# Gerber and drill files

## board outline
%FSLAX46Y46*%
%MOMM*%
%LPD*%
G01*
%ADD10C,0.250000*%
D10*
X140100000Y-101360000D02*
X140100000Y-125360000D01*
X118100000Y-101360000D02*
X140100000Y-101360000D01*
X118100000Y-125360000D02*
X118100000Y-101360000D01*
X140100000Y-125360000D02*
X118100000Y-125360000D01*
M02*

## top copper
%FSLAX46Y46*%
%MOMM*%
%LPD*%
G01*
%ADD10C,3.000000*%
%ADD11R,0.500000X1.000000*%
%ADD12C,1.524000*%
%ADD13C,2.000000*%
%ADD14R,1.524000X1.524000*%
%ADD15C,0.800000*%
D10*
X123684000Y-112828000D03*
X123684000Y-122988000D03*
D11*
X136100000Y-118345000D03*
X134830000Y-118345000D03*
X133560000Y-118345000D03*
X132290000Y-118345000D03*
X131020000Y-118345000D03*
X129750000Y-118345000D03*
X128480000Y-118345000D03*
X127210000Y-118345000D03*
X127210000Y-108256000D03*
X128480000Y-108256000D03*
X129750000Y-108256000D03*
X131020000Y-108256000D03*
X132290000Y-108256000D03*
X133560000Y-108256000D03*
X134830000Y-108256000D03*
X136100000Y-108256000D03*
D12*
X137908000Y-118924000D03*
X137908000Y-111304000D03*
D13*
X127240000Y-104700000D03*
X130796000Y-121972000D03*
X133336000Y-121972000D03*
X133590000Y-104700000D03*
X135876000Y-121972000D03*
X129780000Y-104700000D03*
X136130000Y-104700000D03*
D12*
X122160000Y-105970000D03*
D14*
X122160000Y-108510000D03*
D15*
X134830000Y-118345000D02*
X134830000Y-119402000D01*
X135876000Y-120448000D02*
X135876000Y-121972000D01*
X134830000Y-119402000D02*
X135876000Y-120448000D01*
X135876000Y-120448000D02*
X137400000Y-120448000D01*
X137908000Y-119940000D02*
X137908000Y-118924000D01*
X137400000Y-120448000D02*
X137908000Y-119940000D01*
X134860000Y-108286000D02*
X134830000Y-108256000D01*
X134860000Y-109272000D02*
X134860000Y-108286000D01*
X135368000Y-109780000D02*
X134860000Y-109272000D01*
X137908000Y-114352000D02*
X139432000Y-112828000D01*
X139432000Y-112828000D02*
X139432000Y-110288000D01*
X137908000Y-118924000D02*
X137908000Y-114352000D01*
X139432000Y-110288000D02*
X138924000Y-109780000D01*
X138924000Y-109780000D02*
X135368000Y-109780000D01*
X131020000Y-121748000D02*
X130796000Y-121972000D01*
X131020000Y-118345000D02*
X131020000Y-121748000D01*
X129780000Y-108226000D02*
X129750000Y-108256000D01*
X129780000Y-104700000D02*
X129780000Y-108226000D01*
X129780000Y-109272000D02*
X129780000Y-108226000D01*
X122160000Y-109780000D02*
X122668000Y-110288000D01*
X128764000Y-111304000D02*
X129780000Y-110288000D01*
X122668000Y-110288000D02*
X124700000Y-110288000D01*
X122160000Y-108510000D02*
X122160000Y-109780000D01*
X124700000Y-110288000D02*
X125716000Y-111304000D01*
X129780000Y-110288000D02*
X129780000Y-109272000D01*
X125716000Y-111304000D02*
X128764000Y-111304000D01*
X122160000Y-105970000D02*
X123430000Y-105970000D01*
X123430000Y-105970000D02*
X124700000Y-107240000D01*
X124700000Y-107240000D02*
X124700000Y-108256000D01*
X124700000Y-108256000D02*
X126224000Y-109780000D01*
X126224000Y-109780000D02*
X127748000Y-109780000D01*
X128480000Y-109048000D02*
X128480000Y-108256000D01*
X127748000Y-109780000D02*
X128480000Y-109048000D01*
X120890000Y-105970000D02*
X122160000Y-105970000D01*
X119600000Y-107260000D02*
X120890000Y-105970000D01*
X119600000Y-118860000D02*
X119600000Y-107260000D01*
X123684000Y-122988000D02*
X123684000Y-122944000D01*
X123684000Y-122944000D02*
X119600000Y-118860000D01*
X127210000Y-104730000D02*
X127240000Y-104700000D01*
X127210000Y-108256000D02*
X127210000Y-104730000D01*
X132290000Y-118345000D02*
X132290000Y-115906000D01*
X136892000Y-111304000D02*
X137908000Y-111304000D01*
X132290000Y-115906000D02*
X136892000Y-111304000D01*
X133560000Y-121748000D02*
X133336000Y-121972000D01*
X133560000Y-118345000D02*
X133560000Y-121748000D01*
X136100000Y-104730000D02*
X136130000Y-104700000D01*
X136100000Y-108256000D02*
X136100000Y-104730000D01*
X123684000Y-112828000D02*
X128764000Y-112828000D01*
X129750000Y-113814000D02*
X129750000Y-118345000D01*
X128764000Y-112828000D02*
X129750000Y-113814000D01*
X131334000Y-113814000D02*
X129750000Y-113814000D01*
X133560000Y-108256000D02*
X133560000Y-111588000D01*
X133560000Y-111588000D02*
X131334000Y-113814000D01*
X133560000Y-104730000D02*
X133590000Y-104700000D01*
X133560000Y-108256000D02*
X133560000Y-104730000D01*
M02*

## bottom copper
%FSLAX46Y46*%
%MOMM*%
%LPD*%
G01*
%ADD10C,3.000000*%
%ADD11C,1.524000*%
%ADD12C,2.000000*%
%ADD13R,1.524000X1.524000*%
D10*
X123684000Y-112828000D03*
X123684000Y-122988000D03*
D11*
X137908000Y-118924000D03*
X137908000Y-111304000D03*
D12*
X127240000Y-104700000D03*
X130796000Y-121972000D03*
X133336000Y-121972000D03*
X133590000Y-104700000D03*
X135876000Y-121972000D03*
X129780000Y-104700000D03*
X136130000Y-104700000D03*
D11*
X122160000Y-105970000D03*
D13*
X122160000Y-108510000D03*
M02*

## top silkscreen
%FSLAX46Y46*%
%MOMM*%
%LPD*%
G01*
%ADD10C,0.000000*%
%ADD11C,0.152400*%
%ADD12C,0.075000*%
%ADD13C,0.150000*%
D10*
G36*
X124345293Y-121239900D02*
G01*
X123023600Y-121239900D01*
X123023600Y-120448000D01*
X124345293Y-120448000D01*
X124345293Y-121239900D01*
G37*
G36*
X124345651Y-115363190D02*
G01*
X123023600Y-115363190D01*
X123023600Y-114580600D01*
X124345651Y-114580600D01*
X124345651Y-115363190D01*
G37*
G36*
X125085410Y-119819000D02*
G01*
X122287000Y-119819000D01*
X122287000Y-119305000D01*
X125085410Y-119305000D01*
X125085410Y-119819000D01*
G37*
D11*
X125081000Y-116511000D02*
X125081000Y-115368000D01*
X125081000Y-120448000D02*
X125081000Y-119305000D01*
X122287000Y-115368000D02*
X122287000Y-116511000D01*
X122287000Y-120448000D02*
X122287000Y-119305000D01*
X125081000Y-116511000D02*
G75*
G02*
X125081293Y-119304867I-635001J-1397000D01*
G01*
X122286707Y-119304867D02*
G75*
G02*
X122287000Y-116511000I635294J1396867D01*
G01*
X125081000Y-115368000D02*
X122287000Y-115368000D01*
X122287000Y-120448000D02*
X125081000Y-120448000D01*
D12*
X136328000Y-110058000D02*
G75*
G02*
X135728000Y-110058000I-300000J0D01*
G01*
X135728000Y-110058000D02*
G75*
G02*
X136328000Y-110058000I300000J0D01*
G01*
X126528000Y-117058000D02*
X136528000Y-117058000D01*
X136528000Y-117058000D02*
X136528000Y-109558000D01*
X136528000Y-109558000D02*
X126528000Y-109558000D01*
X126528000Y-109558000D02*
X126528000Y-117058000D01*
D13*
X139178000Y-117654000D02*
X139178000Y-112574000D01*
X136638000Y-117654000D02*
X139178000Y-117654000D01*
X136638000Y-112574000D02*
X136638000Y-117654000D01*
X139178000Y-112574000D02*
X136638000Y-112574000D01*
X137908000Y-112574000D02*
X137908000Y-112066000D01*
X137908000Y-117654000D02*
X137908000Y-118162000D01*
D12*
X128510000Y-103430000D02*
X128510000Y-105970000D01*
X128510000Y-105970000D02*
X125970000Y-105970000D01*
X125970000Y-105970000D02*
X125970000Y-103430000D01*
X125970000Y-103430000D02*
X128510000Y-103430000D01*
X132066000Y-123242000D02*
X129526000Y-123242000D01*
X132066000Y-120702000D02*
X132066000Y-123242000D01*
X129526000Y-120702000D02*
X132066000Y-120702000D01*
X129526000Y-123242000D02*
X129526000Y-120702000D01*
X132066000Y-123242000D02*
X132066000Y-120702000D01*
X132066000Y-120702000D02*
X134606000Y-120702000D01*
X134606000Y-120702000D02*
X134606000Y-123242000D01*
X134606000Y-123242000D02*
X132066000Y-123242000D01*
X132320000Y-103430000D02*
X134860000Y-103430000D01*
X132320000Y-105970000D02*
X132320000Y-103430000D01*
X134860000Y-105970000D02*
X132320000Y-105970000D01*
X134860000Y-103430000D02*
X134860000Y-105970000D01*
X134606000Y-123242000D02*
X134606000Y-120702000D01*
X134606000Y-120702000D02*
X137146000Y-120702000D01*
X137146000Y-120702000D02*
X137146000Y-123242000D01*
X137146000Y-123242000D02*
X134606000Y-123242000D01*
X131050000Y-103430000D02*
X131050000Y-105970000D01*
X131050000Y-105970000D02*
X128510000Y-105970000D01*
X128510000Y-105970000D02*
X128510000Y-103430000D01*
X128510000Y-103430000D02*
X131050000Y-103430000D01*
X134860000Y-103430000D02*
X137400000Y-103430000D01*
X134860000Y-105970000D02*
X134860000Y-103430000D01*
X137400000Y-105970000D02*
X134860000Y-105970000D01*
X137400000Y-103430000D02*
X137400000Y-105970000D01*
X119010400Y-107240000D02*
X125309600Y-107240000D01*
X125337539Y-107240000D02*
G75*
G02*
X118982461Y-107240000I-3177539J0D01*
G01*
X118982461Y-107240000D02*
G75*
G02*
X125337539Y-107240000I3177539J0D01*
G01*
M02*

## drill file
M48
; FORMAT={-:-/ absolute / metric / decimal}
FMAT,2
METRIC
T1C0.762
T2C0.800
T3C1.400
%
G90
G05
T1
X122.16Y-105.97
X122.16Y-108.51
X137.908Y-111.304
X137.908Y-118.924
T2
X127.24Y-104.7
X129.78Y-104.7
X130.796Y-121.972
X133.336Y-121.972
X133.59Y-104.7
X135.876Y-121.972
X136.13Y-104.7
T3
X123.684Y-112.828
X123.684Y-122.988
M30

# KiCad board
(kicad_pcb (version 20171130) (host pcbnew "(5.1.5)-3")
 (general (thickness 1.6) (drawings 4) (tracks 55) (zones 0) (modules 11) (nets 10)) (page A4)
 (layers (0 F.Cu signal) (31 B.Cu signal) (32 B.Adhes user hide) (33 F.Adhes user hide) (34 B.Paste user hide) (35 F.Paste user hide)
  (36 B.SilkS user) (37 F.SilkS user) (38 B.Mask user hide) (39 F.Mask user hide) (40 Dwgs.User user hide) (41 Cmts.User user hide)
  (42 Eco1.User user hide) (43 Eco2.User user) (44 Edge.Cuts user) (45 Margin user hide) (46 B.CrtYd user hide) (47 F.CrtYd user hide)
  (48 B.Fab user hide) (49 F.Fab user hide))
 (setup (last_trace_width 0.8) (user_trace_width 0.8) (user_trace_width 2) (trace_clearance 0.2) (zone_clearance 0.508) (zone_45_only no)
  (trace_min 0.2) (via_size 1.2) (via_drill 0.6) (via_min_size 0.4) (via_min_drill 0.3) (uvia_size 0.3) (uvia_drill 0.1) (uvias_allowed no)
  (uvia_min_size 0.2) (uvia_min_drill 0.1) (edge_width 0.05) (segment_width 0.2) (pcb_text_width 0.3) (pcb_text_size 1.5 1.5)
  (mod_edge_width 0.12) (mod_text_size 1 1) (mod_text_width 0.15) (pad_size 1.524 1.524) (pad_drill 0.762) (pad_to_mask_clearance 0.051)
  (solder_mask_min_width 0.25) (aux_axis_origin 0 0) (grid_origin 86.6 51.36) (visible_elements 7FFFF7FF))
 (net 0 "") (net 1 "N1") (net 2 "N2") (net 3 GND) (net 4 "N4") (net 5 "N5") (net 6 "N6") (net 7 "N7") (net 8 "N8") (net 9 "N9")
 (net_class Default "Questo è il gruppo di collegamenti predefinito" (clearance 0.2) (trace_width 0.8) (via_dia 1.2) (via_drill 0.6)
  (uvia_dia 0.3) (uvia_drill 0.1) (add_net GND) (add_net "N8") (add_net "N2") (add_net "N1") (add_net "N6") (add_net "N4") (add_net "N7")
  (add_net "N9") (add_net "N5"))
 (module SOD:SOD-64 (layer F.Cu) (at 123.684 117.908 90)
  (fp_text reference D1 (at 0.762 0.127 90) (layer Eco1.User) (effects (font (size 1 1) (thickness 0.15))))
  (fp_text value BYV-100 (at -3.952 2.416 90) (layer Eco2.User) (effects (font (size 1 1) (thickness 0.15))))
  (fp_poly (pts (xy -3.3319 -0.6604) (xy -2.54 -0.6604) (xy -2.54 0.661293) (xy -3.3319 0.661293)) (layer F.SilkS) (width 0))
  (fp_poly (pts (xy 2.54481 -0.6604) (xy 3.3274 -0.6604) (xy 3.3274 0.661651) (xy 2.54481 0.661651)) (layer F.SilkS) (width 0))
  (fp_poly (pts (xy -1.911 -1.397) (xy -1.397 -1.397) (xy -1.397 1.40141) (xy -1.911 1.40141)) (layer F.SilkS) (width 0))
  (fp_line (start 1.397 1.397) (end 2.54 1.397) (layer F.SilkS) (width 0.1524))
  (fp_line (start -2.54 1.397) (end -1.397 1.397) (layer F.SilkS) (width 0.1524))
  (fp_line (start 2.54 -1.397) (end 1.397 -1.397) (layer F.SilkS) (width 0.1524))
  (fp_line (start -2.54 -1.397) (end -1.397 -1.397) (layer F.SilkS) (width 0.1524))
  (fp_arc (start 0 0.761999) (end 1.397 1.397) (angle 131.1) (layer F.SilkS) (width 0.1524))
  (fp_arc (start 0 -0.761999) (end 1.397 -1.397) (angle -131.1) (layer F.SilkS) (width 0.1524))
  (fp_line (start 2.54 1.397) (end 2.54 -1.397) (layer F.SilkS) (width 0.1524))
  (fp_line (start -2.54 -1.397) (end -2.54 1.397) (layer F.SilkS) (width 0.1524))
  (pad 2 thru_hole circle (at 5.08 0 90) (size 3 3) (drill 1.4) (layers *.Cu *.Mask) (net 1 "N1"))
  (pad 1 thru_hole circle (at -5.08 0 90) (size 3 3) (drill 1.4) (layers *.Cu *.Mask) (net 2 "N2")))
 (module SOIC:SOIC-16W (layer F.Cu) (at 136.1 108.256 180)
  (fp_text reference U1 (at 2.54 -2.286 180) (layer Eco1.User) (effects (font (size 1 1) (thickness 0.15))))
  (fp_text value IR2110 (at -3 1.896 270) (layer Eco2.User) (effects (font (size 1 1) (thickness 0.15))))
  (fp_circle (center 0.072 -1.802) (end 0.372 -1.802) (layer F.SilkS) (width 0.075))
  (fp_line (start 9.572 -8.802) (end -0.428 -8.802) (layer F.SilkS) (width 0.075))
  (fp_line (start -0.428 -8.802) (end -0.428 -1.302) (layer F.SilkS) (width 0.075))
  (fp_line (start -0.428 -1.302) (end 9.572 -1.302) (layer F.SilkS) (width 0.075))
  (fp_line (start 9.572 -1.302) (end 9.572 -8.802) (layer F.SilkS) (width 0.075))
  (pad 16 smd rect (at 0 -10.089 180) (size 0.5 1) (layers F.Cu F.Paste F.Mask))
  (pad 15 smd rect (at 1.27 -10.089 180) (size 0.5 1) (layers F.Cu F.Paste F.Mask) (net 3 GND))
  (pad 14 smd rect (at 2.54 -10.089 180) (size 0.5 1) (layers F.Cu F.Paste F.Mask) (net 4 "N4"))
  (pad 13 smd rect (at 3.81 -10.089 180) (size 0.5 1) (layers F.Cu F.Paste F.Mask) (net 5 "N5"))
  (pad 12 smd rect (at 5.08 -10.089 180) (size 0.5 1) (layers F.Cu F.Paste F.Mask) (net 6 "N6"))
  (pad 11 smd rect (at 6.35 -10.089 180) (size 0.5 1) (layers F.Cu F.Paste F.Mask) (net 1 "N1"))
  (pad 10 smd rect (at 7.62 -10.089 180) (size 0.5 1) (layers F.Cu F.Paste F.Mask))
  (pad 9 smd rect (at 8.89 -10.089 180) (size 0.5 1) (layers F.Cu F.Paste F.Mask))
  (pad 8 smd rect (at 8.89 0 180) (size 0.5 1) (layers F.Cu F.Paste F.Mask) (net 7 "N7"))
  (pad 7 smd rect (at 7.62 0 180) (size 0.5 1) (layers F.Cu F.Paste F.Mask) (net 2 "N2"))
  (pad 6 smd rect (at 6.35 0 180) (size 0.5 1) (layers F.Cu F.Paste F.Mask) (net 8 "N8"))
  (pad 5 smd rect (at 5.08 0 180) (size 0.5 1) (layers F.Cu F.Paste F.Mask))
  (pad 4 smd rect (at 3.81 0 180) (size 0.5 1) (layers F.Cu F.Paste F.Mask))
  (pad 3 smd rect (at 2.54 0 180) (size 0.5 1) (layers F.Cu F.Paste F.Mask) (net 1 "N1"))
  (pad 2 smd rect (at 1.27 0 180) (size 0.5 1) (layers F.Cu F.Paste F.Mask) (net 3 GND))
  (pad 1 smd rect (at 0 0 180) (size 0.5 1) (layers F.Cu F.Paste F.Mask) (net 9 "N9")))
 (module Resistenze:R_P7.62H (layer F.Cu) (at 137.908 115.114 270)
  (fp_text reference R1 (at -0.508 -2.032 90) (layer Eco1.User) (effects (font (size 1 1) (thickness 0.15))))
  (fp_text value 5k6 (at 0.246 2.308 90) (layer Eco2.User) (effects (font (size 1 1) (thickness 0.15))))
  (fp_line (start 2.54 -1.27) (end -2.54 -1.27) (layer F.SilkS) (width 0.15))
  (fp_line (start 2.54 1.27) (end 2.54 -1.27) (layer F.SilkS) (width 0.15))
  (fp_line (start -2.54 1.27) (end 2.54 1.27) (layer F.SilkS) (width 0.15))
  (fp_line (start -2.54 -1.27) (end -2.54 1.27) (layer F.SilkS) (width 0.15))
  (fp_line (start -2.54 0) (end -3.048 0) (layer F.SilkS) (width 0.15))
  (fp_line (start 2.54 0) (end 3.048 0) (layer F.SilkS) (width 0.15))
  (pad 2 thru_hole circle (at 3.81 0 270) (size 1.524 1.524) (drill 0.762) (layers *.Cu *.Mask) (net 3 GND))
  (pad 1 thru_hole circle (at -3.81 0 270) (size 1.524 1.524) (drill 0.762) (layers *.Cu *.Mask) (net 5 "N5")))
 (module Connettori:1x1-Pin (layer F.Cu) (at 127.24 104.7 270)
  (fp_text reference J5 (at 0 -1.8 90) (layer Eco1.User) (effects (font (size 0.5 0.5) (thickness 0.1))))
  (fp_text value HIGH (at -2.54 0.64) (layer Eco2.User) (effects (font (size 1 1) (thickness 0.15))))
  (fp_line (start -1.27 -1.27) (end 1.27 -1.27) (layer F.SilkS) (width 0.075))
  (fp_line (start 1.27 -1.27) (end 1.27 1.27) (layer F.SilkS) (width 0.075))
  (fp_line (start 1.27 1.27) (end -1.27 1.27) (layer F.SilkS) (width 0.075))
  (fp_line (start -1.27 1.27) (end -1.27 -1.27) (layer F.SilkS) (width 0.075))
  (pad 1 thru_hole circle (at 0 0 270) (size 2 2) (drill 0.8) (layers *.Cu *.Mask) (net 7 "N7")))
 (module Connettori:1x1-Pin (layer F.Cu) (at 130.796 121.972 90)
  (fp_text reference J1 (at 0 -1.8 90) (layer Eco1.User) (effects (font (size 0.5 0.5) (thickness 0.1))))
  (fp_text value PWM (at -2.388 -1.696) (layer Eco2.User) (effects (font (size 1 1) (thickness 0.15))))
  (fp_line (start -1.27 1.27) (end -1.27 -1.27) (layer F.SilkS) (width 0.075))
  (fp_line (start 1.27 1.27) (end -1.27 1.27) (layer F.SilkS) (width 0.075))
  (fp_line (start 1.27 -1.27) (end 1.27 1.27) (layer F.SilkS) (width 0.075))
  (fp_line (start -1.27 -1.27) (end 1.27 -1.27) (layer F.SilkS) (width 0.075))
  (pad 1 thru_hole circle (at 0 0 90) (size 2 2) (drill 0.8) (layers *.Cu *.Mask) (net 6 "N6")))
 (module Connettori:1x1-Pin (layer F.Cu) (at 133.336 121.972 90)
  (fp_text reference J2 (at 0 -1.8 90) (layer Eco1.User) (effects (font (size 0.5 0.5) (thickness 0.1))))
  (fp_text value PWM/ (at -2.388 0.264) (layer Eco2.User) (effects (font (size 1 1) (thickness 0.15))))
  (fp_line (start -1.27 -1.27) (end 1.27 -1.27) (layer F.SilkS) (width 0.075))
  (fp_line (start 1.27 -1.27) (end 1.27 1.27) (layer F.SilkS) (width 0.075))
  (fp_line (start 1.27 1.27) (end -1.27 1.27) (layer F.SilkS) (width 0.075))
  (fp_line (start -1.27 1.27) (end -1.27 -1.27) (layer F.SilkS) (width 0.075))
  (pad 1 thru_hole circle (at 0 0 90) (size 2 2) (drill 0.8) (layers *.Cu *.Mask) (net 4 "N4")))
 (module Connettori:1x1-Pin (layer F.Cu) (at 133.59 104.7 270)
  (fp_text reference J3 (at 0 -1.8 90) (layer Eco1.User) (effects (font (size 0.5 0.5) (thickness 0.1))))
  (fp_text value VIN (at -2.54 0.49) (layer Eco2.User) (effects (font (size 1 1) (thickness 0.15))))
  (fp_line (start -1.27 1.27) (end -1.27 -1.27) (layer F.SilkS) (width 0.075))
  (fp_line (start 1.27 1.27) (end -1.27 1.27) (layer F.SilkS) (width 0.075))
  (fp_line (start 1.27 -1.27) (end 1.27 1.27) (layer F.SilkS) (width 0.075))
  (fp_line (start -1.27 -1.27) (end 1.27 -1.27) (layer F.SilkS) (width 0.075))
  (pad 1 thru_hole circle (at 0 0 270) (size 2 2) (drill 0.8) (layers *.Cu *.Mask) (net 1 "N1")))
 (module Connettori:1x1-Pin (layer F.Cu) (at 135.876 121.972 90)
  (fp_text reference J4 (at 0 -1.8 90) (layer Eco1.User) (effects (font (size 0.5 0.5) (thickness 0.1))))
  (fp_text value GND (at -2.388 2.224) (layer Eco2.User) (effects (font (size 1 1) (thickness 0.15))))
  (fp_line (start -1.27 -1.27) (end 1.27 -1.27) (layer F.SilkS) (width 0.075))
  (fp_line (start 1.27 -1.27) (end 1.27 1.27) (layer F.SilkS) (width 0.075))
  (fp_line (start 1.27 1.27) (end -1.27 1.27) (layer F.SilkS) (width 0.075))
  (fp_line (start -1.27 1.27) (end -1.27 -1.27) (layer F.SilkS) (width 0.075))
  (pad 1 thru_hole circle (at 0 0 90) (size 2 2) (drill 0.8) (layers *.Cu *.Mask) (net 3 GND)))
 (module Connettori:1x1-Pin (layer F.Cu) (at 129.78 104.7 270)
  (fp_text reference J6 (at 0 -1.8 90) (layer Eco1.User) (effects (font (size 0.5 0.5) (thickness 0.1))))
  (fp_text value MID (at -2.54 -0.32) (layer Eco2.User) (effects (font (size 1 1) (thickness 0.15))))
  (fp_line (start -1.27 -1.27) (end 1.27 -1.27) (layer F.SilkS) (width 0.075))
  (fp_line (start 1.27 -1.27) (end 1.27 1.27) (layer F.SilkS) (width 0.075))
  (fp_line (start 1.27 1.27) (end -1.27 1.27) (layer F.SilkS) (width 0.075))
  (fp_line (start -1.27 1.27) (end -1.27 -1.27) (layer F.SilkS) (width 0.075))
  (pad 1 thru_hole circle (at 0 0 270) (size 2 2) (drill 0.8) (layers *.Cu *.Mask) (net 8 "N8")))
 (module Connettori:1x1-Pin (layer F.Cu) (at 136.13 104.7 270)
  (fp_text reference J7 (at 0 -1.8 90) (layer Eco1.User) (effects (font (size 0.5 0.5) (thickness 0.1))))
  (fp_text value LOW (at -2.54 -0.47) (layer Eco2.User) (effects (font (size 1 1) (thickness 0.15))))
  (fp_line (start -1.27 1.27) (end -1.27 -1.27) (layer F.SilkS) (width 0.075))
  (fp_line (start 1.27 1.27) (end -1.27 1.27) (layer F.SilkS) (width 0.075))
  (fp_line (start 1.27 -1.27) (end 1.27 1.27) (layer F.SilkS) (width 0.075))
  (fp_line (start -1.27 -1.27) (end 1.27 -1.27) (layer F.SilkS) (width 0.075))
  (pad 1 thru_hole circle (at 0 0 270) (size 2 2) (drill 0.8) (layers *.Cu *.Mask) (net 9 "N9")))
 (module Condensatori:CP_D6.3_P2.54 (layer F.Cu) (at 122.16 107.24 90)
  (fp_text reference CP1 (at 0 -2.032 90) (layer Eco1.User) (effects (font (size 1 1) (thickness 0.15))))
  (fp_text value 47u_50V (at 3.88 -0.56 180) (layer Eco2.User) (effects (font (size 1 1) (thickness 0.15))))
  (fp_line (start 0 -3.1496) (end 0 3.1496) (layer F.SilkS) (width 0.075))
  (fp_circle (center 0 0) (end 3.175 -0.127) (layer F.SilkS) (width 0.075))
  (pad 2 thru_hole circle (at 1.27 0 90) (size 1.524 1.524) (drill 0.762) (layers *.Cu *.Mask) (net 2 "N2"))
  (pad 1 thru_hole rect (at -1.27 0 90) (size 1.524 1.524) (drill 0.762) (layers *.Cu *.Mask) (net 8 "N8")))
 (gr_line (start 140.1 101.36) (end 140.1 125.36) (layer Edge.Cuts) (width 0.25))
 (gr_line (start 118.1 101.36) (end 140.1 101.36) (layer Edge.Cuts) (width 0.25))
 (gr_line (start 118.1 125.36) (end 118.1 101.36) (layer Edge.Cuts) (width 0.25))
 (gr_line (start 140.1 125.36) (end 118.1 125.36) (layer Edge.Cuts) (width 0.25))
 (segment (start 134.83 118.345) (end 134.83 119.402) (width 0.8) (layer F.Cu) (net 3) (status 10))
 (segment (start 135.876 120.448) (end 135.876 121.972) (width 0.8) (layer F.Cu) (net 3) (status 20))
 (segment (start 134.83 119.402) (end 135.876 120.448) (width 0.8) (layer F.Cu) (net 3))
 (segment (start 135.876 120.448) (end 137.4 120.448) (width 0.8) (layer F.Cu) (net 3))
 (segment (start 137.908 119.94) (end 137.908 118.924) (width 0.8) (layer F.Cu) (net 3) (status 20))
 (segment (start 137.4 120.448) (end 137.908 119.94) (width 0.8) (layer F.Cu) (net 3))
 (segment (start 134.86 108.286) (end 134.83 108.256) (width 0.8) (layer F.Cu) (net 3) (status 30))
 (segment (start 134.86 109.272) (end 134.86 108.286) (width 0.8) (layer F.Cu) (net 3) (status 20))
 (segment (start 135.368 109.78) (end 134.86 109.272) (width 0.8) (layer F.Cu) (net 3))
 (segment (start 137.908 114.352) (end 139.432 112.828) (width 0.8) (layer F.Cu) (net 3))
 (segment (start 139.432 112.828) (end 139.432 110.288) (width 0.8) (layer F.Cu) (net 3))
 (segment (start 137.908 118.924) (end 137.908 114.352) (width 0.8) (layer F.Cu) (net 3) (status 10))
 (segment (start 139.432 110.288) (end 138.924 109.78) (width 0.8) (layer F.Cu) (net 3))
 (segment (start 138.924 109.78) (end 135.368 109.78) (width 0.8) (layer F.Cu) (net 3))
 (segment (start 131.02 121.748) (end 130.796 121.972) (width 0.8) (layer F.Cu) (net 6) (status 30))
 (segment (start 131.02 118.345) (end 131.02 121.748) (width 0.8) (layer F.Cu) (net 6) (status 30))
 (segment (start 129.78 108.226) (end 129.75 108.256) (width 0.8) (layer F.Cu) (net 8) (status 30))
 (segment (start 129.78 104.7) (end 129.78 108.226) (width 0.8) (layer F.Cu) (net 8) (status 30))
 (segment (start 129.78 109.272) (end 129.78 108.226) (width 0.8) (layer F.Cu) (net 8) (status 20))
 (segment (start 122.16 109.78) (end 122.668 110.288) (width 0.8) (layer F.Cu) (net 8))
 (segment (start 128.764 111.304) (end 129.78 110.288) (width 0.8) (layer F.Cu) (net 8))
 (segment (start 122.668 110.288) (end 124.7 110.288) (width 0.8) (layer F.Cu) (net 8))
 (segment (start 122.16 108.51) (end 122.16 109.78) (width 0.8) (layer F.Cu) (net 8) (status 10))
 (segment (start 124.7 110.288) (end 125.716 111.304) (width 0.8) (layer F.Cu) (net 8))
 (segment (start 129.78 110.288) (end 129.78 109.272) (width 0.8) (layer F.Cu) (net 8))
 (segment (start 125.716 111.304) (end 128.764 111.304) (width 0.8) (layer F.Cu) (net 8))
 (segment (start 122.16 105.97) (end 123.43 105.97) (width 0.8) (layer F.Cu) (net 2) (status 10))
 (segment (start 123.43 105.97) (end 124.7 107.24) (width 0.8) (layer F.Cu) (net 2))
 (segment (start 124.7 107.24) (end 124.7 108.256) (width 0.8) (layer F.Cu) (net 2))
 (segment (start 124.7 108.256) (end 126.224 109.78) (width 0.8) (layer F.Cu) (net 2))
 (segment (start 126.224 109.78) (end 127.748 109.78) (width 0.8) (layer F.Cu) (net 2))
 (segment (start 128.48 109.048) (end 128.48 108.256) (width 0.8) (layer F.Cu) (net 2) (status 20))
 (segment (start 127.748 109.78) (end 128.48 109.048) (width 0.8) (layer F.Cu) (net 2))
 (segment (start 120.89 105.97) (end 122.16 105.97) (width 0.8) (layer F.Cu) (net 2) (status 20))
 (segment (start 119.6 107.26) (end 120.89 105.97) (width 0.8) (layer F.Cu) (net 2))
 (segment (start 119.6 118.86) (end 119.6 107.26) (width 0.8) (layer F.Cu) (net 2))
 (segment (start 123.684 122.988) (end 123.684 122.944) (width 0.8) (layer F.Cu) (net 2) (status 30))
 (segment (start 123.684 122.944) (end 119.6 118.86) (width 0.8) (layer F.Cu) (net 2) (status 10))
 (segment (start 127.21 104.73) (end 127.24 104.7) (width 0.8) (layer F.Cu) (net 7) (status 30))
 (segment (start 127.21 108.256) (end 127.21 104.73) (width 0.8) (layer F.Cu) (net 7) (status 30))
 (segment (start 132.29 118.345) (end 132.29 115.906) (width 0.8) (layer F.Cu) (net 5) (status 10))
 (segment (start 136.892 111.304) (end 137.908 111.304) (width 0.8) (layer F.Cu) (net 5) (status 20))
 (segment (start 132.29 115.906) (end 136.892 111.304) (width 0.8) (layer F.Cu) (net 5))
 (segment (start 133.56 121.748) (end 133.336 121.972) (width 0.8) (layer F.Cu) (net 4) (status 30))
 (segment (start 133.56 118.345) (end 133.56 121.748) (width 0.8) (layer F.Cu) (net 4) (status 30))
 (segment (start 136.1 104.73) (end 136.13 104.7) (width 0.8) (layer F.Cu) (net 9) (status 30))
 (segment (start 136.1 108.256) (end 136.1 104.73) (width 0.8) (layer F.Cu) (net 9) (status 30))
 (segment (start 123.684 112.828) (end 128.764 112.828) (width 0.8) (layer F.Cu) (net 1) (status 10))
 (segment (start 129.75 113.814) (end 129.75 118.345) (width 0.8) (layer F.Cu) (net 1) (status 20))
 (segment (start 128.764 112.828) (end 129.75 113.814) (width 0.8) (layer F.Cu) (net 1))
 (segment (start 131.334 113.814) (end 129.75 113.814) (width 0.8) (layer F.Cu) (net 1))
 (segment (start 133.56 108.256) (end 133.56 111.588) (width 0.8) (layer F.Cu) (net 1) (status 10))
 (segment (start 133.56 111.588) (end 131.334 113.814) (width 0.8) (layer F.Cu) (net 1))
 (segment (start 133.56 104.73) (end 133.59 104.7) (width 0.8) (layer F.Cu) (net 1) (status 30))
 (segment (start 133.56 108.256) (end 133.56 104.73) (width 0.8) (layer F.Cu) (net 1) (status 30)))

